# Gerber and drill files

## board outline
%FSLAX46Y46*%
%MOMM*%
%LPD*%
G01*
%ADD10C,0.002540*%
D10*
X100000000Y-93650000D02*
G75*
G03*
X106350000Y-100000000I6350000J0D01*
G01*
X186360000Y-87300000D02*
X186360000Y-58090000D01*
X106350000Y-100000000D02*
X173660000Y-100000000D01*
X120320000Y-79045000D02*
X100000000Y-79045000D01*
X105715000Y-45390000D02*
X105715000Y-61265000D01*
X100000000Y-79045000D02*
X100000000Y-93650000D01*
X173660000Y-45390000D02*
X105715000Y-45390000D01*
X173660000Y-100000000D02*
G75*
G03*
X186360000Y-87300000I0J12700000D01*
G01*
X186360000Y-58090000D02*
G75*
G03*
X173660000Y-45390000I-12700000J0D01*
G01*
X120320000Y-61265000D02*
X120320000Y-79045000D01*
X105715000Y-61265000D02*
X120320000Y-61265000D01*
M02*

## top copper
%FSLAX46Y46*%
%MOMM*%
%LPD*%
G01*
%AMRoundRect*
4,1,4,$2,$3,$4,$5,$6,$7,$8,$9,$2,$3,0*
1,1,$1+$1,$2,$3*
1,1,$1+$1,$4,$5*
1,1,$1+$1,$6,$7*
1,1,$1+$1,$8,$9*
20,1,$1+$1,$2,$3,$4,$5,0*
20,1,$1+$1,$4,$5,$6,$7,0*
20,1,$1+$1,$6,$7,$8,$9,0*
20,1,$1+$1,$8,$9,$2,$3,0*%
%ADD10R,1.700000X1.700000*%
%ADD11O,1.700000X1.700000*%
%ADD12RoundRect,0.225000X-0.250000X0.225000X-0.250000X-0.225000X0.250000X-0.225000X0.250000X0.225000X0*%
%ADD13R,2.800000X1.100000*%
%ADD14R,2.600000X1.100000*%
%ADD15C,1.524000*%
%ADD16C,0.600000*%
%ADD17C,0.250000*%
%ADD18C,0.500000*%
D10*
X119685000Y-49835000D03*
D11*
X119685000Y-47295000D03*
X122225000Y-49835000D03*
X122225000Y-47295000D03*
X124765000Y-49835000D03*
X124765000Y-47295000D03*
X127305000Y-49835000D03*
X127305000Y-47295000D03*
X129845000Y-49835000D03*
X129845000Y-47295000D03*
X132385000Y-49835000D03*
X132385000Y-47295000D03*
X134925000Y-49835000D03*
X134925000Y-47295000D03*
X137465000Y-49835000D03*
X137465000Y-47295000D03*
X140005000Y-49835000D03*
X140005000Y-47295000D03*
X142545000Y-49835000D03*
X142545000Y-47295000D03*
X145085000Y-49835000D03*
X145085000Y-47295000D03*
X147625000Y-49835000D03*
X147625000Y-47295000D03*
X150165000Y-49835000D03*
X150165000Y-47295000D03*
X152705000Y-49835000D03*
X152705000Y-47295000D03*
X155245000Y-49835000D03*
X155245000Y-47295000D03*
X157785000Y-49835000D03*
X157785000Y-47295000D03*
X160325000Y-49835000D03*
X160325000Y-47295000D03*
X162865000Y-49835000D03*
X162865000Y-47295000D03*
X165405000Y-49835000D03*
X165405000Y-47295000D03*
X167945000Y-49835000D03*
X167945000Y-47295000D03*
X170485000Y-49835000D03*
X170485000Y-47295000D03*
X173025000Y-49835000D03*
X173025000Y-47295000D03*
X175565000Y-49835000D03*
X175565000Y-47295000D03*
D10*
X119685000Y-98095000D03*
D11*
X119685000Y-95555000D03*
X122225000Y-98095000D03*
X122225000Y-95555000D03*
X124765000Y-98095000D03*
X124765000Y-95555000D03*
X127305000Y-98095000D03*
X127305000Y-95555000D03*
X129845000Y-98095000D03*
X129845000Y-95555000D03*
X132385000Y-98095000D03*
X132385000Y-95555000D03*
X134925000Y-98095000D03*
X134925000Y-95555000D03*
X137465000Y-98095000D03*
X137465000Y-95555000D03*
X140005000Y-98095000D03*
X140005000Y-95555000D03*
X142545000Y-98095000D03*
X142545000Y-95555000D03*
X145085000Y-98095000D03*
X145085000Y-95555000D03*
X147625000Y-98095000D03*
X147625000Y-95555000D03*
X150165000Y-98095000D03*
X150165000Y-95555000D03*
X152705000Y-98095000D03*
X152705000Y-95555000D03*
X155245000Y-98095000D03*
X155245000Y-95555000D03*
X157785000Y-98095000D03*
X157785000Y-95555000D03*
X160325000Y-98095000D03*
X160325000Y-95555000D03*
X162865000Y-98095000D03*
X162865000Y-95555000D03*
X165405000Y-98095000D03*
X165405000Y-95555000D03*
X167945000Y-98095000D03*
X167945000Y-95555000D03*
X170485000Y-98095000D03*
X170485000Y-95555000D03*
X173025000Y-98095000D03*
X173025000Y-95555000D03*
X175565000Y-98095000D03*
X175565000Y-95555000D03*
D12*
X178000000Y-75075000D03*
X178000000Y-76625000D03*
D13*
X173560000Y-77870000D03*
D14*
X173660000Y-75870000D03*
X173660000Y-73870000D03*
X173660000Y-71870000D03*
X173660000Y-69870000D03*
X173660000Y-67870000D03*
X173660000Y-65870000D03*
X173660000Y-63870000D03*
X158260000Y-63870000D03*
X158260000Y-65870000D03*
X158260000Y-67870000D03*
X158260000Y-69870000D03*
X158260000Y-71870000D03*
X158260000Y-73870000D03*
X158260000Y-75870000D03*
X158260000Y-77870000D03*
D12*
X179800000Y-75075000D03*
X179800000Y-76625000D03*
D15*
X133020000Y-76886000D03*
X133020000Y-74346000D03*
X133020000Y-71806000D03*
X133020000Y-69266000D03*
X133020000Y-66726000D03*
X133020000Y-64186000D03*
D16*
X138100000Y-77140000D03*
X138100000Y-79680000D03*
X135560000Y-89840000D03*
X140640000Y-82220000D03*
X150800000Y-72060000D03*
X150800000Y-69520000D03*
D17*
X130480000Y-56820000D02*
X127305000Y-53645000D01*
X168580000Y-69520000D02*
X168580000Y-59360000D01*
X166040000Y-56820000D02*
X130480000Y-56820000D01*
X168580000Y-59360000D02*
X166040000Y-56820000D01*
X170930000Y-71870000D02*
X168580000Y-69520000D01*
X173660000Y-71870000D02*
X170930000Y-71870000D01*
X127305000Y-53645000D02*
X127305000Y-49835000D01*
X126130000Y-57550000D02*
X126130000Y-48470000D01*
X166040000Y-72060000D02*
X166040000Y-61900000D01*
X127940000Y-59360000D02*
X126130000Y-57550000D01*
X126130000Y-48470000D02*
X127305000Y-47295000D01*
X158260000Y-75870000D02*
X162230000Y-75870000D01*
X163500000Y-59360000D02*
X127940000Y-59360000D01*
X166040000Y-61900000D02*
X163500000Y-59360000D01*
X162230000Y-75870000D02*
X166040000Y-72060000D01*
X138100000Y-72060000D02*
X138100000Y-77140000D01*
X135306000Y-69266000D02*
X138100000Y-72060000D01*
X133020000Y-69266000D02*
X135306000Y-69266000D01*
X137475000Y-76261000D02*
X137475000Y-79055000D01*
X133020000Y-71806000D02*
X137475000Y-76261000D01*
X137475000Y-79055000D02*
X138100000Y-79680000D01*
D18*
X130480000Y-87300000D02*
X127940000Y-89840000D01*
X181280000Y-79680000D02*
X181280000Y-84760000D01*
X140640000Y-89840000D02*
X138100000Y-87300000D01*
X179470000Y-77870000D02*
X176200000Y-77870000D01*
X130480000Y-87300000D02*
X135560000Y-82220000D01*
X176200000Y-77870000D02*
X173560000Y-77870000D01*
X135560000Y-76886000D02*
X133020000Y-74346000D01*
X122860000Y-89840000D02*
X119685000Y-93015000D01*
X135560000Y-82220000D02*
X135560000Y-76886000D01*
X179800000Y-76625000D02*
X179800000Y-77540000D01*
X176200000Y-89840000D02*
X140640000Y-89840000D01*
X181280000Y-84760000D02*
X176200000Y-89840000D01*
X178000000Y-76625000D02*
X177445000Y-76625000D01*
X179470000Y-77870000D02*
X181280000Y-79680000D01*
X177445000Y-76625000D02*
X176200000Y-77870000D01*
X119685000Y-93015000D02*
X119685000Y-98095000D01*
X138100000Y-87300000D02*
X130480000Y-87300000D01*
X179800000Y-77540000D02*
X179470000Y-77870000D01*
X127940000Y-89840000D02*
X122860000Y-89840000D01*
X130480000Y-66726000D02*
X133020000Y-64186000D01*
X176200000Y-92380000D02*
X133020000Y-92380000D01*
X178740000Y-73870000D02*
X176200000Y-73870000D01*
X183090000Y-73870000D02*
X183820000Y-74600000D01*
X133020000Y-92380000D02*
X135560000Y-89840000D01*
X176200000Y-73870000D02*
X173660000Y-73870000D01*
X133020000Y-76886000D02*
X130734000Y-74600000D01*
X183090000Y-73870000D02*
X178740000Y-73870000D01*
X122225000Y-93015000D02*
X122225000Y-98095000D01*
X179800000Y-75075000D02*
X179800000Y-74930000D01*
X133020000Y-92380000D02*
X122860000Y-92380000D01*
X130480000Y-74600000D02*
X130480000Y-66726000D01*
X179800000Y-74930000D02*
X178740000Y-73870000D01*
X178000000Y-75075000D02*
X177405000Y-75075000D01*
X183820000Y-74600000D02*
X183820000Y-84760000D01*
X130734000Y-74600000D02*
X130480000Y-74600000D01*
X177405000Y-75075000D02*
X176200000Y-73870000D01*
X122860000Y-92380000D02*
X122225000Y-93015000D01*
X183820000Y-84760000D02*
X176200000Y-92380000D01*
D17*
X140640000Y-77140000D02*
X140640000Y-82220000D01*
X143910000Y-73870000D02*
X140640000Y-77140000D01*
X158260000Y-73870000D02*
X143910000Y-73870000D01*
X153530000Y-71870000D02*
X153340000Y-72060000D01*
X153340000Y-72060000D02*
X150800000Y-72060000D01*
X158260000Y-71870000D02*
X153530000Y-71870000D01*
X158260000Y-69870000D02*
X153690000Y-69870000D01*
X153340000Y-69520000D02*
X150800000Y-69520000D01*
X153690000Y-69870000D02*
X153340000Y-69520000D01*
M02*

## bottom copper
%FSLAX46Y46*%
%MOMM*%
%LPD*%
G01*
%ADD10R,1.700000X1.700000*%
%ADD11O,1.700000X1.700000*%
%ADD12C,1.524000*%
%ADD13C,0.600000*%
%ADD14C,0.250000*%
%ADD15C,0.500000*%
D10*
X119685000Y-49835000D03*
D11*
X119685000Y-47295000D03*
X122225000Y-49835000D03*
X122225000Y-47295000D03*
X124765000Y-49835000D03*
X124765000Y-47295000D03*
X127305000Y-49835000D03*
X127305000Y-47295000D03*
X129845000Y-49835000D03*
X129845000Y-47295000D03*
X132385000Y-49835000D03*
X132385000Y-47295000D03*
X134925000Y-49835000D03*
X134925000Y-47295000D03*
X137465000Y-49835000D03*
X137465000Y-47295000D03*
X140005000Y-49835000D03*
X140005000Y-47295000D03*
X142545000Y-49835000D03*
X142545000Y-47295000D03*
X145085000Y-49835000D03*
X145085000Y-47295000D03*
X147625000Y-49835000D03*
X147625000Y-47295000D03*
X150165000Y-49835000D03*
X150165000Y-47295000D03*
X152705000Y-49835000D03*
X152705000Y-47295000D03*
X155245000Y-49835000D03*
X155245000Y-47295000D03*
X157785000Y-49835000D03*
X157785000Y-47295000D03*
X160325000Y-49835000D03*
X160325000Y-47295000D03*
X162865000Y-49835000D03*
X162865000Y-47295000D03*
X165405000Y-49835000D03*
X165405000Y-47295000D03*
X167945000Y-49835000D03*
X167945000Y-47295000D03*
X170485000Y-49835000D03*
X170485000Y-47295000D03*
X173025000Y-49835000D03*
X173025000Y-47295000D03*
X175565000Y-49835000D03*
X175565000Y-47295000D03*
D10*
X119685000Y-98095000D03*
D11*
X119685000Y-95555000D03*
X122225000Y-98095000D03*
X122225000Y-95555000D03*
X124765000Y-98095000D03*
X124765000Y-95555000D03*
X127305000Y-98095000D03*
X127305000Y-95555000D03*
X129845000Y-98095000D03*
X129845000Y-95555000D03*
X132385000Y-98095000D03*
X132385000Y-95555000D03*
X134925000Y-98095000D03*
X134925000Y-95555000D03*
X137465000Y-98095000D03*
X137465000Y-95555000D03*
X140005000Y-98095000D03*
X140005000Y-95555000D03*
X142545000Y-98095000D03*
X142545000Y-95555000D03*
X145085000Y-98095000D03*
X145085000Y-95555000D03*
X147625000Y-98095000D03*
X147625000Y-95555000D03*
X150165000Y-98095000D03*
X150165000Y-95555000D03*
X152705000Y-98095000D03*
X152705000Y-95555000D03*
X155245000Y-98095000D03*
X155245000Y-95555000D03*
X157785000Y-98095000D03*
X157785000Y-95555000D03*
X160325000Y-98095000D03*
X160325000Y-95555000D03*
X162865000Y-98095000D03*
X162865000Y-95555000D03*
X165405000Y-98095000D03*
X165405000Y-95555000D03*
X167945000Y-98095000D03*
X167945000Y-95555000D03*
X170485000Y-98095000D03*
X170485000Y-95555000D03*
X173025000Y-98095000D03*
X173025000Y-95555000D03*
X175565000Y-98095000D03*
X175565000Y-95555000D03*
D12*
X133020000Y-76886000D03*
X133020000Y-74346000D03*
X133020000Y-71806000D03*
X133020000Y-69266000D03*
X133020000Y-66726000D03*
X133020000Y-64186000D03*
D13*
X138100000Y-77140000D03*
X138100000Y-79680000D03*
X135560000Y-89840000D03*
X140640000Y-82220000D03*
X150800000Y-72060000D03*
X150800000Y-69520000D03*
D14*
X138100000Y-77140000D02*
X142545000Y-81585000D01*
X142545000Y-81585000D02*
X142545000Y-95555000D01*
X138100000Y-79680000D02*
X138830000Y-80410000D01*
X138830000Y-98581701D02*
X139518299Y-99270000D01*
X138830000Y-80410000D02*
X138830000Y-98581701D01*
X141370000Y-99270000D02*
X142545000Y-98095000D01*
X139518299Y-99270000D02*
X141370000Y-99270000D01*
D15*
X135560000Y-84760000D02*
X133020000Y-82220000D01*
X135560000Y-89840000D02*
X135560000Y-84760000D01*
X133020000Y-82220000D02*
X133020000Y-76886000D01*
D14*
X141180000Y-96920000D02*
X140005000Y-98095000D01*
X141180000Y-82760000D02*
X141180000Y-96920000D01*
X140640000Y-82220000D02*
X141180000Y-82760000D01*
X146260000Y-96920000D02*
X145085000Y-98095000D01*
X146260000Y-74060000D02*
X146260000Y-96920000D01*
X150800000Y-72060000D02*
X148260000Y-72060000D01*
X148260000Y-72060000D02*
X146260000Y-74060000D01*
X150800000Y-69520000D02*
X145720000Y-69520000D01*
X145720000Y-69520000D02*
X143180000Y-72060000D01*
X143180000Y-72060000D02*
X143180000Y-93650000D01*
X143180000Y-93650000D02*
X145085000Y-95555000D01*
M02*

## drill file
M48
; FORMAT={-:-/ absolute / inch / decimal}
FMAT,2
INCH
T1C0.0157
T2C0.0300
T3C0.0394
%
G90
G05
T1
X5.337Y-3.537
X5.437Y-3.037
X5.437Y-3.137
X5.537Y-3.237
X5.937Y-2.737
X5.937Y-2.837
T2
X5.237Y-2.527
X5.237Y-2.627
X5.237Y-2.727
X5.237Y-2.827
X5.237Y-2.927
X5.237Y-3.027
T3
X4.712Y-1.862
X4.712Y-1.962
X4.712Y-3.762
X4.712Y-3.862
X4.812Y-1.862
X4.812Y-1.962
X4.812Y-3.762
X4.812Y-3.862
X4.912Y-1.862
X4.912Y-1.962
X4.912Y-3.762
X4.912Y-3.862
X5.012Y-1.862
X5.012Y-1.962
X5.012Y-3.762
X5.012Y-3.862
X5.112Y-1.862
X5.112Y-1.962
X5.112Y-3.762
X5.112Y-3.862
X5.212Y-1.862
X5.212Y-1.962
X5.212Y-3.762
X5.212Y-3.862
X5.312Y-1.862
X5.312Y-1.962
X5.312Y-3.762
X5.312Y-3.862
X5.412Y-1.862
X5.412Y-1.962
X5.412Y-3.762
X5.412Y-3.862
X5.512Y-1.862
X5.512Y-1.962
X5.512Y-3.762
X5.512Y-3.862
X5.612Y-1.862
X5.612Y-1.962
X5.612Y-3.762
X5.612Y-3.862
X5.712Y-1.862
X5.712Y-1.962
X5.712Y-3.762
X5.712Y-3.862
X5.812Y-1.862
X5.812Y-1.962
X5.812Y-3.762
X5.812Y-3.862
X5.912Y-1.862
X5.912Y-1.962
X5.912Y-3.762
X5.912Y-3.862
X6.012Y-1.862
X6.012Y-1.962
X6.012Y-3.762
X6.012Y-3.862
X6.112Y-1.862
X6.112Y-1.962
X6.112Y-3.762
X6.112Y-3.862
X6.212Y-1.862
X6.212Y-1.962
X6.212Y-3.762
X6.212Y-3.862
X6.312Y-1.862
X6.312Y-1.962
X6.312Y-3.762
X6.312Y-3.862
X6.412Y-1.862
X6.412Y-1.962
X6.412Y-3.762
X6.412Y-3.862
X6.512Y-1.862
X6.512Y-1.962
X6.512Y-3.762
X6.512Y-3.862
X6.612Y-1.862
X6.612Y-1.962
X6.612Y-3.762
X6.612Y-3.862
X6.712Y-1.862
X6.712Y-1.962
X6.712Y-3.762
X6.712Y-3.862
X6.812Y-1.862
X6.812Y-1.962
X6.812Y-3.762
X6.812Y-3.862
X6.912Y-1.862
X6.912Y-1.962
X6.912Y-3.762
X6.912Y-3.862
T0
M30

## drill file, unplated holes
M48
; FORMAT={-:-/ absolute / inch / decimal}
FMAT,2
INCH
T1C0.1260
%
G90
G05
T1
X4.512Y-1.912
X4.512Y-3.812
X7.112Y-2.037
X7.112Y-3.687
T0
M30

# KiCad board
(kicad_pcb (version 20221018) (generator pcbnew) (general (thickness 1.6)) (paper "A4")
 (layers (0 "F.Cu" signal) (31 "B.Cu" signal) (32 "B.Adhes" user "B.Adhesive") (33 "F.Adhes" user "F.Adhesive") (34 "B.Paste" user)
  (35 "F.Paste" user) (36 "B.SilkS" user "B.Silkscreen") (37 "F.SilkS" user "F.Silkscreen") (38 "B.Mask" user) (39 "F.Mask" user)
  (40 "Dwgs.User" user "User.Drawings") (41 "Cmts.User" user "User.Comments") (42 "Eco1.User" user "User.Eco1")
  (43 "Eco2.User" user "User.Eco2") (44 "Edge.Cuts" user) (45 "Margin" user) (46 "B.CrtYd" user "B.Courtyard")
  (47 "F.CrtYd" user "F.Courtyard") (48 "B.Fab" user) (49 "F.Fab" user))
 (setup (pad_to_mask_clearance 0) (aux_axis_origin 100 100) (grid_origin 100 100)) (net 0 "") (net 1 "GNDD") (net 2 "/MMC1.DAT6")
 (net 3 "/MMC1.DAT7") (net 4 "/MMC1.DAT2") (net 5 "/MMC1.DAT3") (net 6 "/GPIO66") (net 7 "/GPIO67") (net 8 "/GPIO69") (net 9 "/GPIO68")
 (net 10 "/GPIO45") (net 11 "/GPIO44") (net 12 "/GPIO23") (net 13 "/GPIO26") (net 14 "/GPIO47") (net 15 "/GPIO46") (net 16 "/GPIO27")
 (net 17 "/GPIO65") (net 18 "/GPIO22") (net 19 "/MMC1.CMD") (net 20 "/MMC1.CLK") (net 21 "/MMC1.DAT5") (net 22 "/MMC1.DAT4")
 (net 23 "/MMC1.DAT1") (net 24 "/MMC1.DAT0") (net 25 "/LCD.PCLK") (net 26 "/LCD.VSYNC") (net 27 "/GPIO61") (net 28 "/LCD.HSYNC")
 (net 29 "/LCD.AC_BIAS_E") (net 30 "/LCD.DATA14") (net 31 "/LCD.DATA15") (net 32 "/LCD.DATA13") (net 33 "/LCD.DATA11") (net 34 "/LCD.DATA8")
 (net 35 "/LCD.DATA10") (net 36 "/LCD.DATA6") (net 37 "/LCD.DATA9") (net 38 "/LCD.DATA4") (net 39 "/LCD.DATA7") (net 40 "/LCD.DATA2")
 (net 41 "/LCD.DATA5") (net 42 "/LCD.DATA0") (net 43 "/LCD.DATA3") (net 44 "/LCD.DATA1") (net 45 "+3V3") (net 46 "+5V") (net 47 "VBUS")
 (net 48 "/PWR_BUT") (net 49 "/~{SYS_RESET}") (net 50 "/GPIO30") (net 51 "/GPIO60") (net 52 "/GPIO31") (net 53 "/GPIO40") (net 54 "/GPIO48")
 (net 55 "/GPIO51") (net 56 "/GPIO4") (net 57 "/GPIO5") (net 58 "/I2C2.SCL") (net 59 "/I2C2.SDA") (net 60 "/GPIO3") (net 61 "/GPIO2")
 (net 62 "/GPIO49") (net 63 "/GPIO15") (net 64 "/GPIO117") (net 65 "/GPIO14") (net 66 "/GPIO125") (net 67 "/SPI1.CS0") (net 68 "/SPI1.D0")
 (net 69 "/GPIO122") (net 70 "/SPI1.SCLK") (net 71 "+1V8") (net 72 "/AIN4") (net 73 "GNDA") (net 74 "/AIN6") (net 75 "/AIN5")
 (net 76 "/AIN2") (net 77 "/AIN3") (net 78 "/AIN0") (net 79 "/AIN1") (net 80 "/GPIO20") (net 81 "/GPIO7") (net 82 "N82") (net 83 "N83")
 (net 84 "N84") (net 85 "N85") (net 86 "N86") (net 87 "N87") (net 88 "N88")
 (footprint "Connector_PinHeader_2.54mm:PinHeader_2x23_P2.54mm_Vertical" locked (layer "F.Cu") (at 119.685 49.835 90)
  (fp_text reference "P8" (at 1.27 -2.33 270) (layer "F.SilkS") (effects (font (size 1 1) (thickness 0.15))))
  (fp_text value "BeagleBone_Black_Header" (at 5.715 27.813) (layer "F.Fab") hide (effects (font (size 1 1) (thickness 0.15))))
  (pad "1" thru_hole rect locked (at 0 0 90) (size 1.7 1.7) (drill 1) (layers "*.Cu" "*.Mask") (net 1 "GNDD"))
  (pad "2" thru_hole oval locked (at 2.54 0 90) (size 1.7 1.7) (drill 1) (layers "*.Cu" "*.Mask") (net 1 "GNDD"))
  (pad "3" thru_hole oval locked (at 0 2.54 90) (size 1.7 1.7) (drill 1) (layers "*.Cu" "*.Mask") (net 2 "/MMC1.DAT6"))
  (pad "4" thru_hole oval locked (at 2.54 2.54 90) (size 1.7 1.7) (drill 1) (layers "*.Cu" "*.Mask") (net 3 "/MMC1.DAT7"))
  (pad "5" thru_hole oval locked (at 0 5.08 90) (size 1.7 1.7) (drill 1) (layers "*.Cu" "*.Mask") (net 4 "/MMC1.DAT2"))
  (pad "6" thru_hole oval locked (at 2.54 5.08 90) (size 1.7 1.7) (drill 1) (layers "*.Cu" "*.Mask") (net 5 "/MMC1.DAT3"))
  (pad "7" thru_hole oval locked (at 0 7.62 90) (size 1.7 1.7) (drill 1) (layers "*.Cu" "*.Mask") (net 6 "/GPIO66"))
  (pad "8" thru_hole oval locked (at 2.54 7.62 90) (size 1.7 1.7) (drill 1) (layers "*.Cu" "*.Mask") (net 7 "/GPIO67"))
  (pad "9" thru_hole oval locked (at 0 10.16 90) (size 1.7 1.7) (drill 1) (layers "*.Cu" "*.Mask") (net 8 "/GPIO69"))
  (pad "10" thru_hole oval locked (at 2.54 10.16 90) (size 1.7 1.7) (drill 1) (layers "*.Cu" "*.Mask") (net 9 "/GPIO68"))
  (pad "11" thru_hole oval locked (at 0 12.7 90) (size 1.7 1.7) (drill 1) (layers "*.Cu" "*.Mask") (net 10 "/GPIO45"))
  (pad "12" thru_hole oval locked (at 2.54 12.7 90) (size 1.7 1.7) (drill 1) (layers "*.Cu" "*.Mask") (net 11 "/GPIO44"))
  (pad "13" thru_hole oval locked (at 0 15.24 90) (size 1.7 1.7) (drill 1) (layers "*.Cu" "*.Mask") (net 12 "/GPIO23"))
  (pad "14" thru_hole oval locked (at 2.54 15.24 90) (size 1.7 1.7) (drill 1) (layers "*.Cu" "*.Mask") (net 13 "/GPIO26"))
  (pad "15" thru_hole oval locked (at 0 17.78 90) (size 1.7 1.7) (drill 1) (layers "*.Cu" "*.Mask") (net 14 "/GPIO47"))
  (pad "16" thru_hole oval locked (at 2.54 17.78 90) (size 1.7 1.7) (drill 1) (layers "*.Cu" "*.Mask") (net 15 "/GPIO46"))
  (pad "17" thru_hole oval locked (at 0 20.32 90) (size 1.7 1.7) (drill 1) (layers "*.Cu" "*.Mask") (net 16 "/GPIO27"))
  (pad "18" thru_hole oval locked (at 2.54 20.32 90) (size 1.7 1.7) (drill 1) (layers "*.Cu" "*.Mask") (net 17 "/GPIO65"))
  (pad "19" thru_hole oval locked (at 0 22.86 90) (size 1.7 1.7) (drill 1) (layers "*.Cu" "*.Mask") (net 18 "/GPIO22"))
  (pad "20" thru_hole oval locked (at 2.54 22.86 90) (size 1.7 1.7) (drill 1) (layers "*.Cu" "*.Mask") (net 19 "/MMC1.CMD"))
  (pad "21" thru_hole oval locked (at 0 25.4 90) (size 1.7 1.7) (drill 1) (layers "*.Cu" "*.Mask") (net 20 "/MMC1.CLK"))
  (pad "22" thru_hole oval locked (at 2.54 25.4 90) (size 1.7 1.7) (drill 1) (layers "*.Cu" "*.Mask") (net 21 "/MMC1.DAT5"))
  (pad "23" thru_hole oval locked (at 0 27.94 90) (size 1.7 1.7) (drill 1) (layers "*.Cu" "*.Mask") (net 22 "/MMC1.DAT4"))
  (pad "24" thru_hole oval locked (at 2.54 27.94 90) (size 1.7 1.7) (drill 1) (layers "*.Cu" "*.Mask") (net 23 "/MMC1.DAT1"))
  (pad "25" thru_hole oval locked (at 0 30.48 90) (size 1.7 1.7) (drill 1) (layers "*.Cu" "*.Mask") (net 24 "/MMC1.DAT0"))
  (pad "26" thru_hole oval locked (at 2.54 30.48 90) (size 1.7 1.7) (drill 1) (layers "*.Cu" "*.Mask") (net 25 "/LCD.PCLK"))
  (pad "27" thru_hole oval locked (at 0 33.02 90) (size 1.7 1.7) (drill 1) (layers "*.Cu" "*.Mask") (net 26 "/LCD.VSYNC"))
  (pad "28" thru_hole oval locked (at 2.54 33.02 90) (size 1.7 1.7) (drill 1) (layers "*.Cu" "*.Mask") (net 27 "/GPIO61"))
  (pad "29" thru_hole oval locked (at 0 35.56 90) (size 1.7 1.7) (drill 1) (layers "*.Cu" "*.Mask") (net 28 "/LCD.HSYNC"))
  (pad "30" thru_hole oval locked (at 2.54 35.56 90) (size 1.7 1.7) (drill 1) (layers "*.Cu" "*.Mask") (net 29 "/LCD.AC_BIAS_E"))
  (pad "31" thru_hole oval locked (at 0 38.1 90) (size 1.7 1.7) (drill 1) (layers "*.Cu" "*.Mask") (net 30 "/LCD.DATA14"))
  (pad "32" thru_hole oval locked (at 2.54 38.1 90) (size 1.7 1.7) (drill 1) (layers "*.Cu" "*.Mask") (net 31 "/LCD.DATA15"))
  (pad "33" thru_hole oval locked (at 0 40.64 90) (size 1.7 1.7) (drill 1) (layers "*.Cu" "*.Mask") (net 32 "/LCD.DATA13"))
  (pad "34" thru_hole oval locked (at 2.54 40.64 90) (size 1.7 1.7) (drill 1) (layers "*.Cu" "*.Mask") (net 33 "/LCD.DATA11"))
  (pad "35" thru_hole oval locked (at 0 43.18 90) (size 1.7 1.7) (drill 1) (layers "*.Cu" "*.Mask") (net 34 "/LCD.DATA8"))
  (pad "36" thru_hole oval locked (at 2.54 43.18 90) (size 1.7 1.7) (drill 1) (layers "*.Cu" "*.Mask") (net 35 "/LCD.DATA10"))
  (pad "37" thru_hole oval locked (at 0 45.72 90) (size 1.7 1.7) (drill 1) (layers "*.Cu" "*.Mask") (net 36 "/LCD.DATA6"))
  (pad "38" thru_hole oval locked (at 2.54 45.72 90) (size 1.7 1.7) (drill 1) (layers "*.Cu" "*.Mask") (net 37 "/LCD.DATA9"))
  (pad "39" thru_hole oval locked (at 0 48.26 90) (size 1.7 1.7) (drill 1) (layers "*.Cu" "*.Mask") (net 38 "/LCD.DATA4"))
  (pad "40" thru_hole oval locked (at 2.54 48.26 90) (size 1.7 1.7) (drill 1) (layers "*.Cu" "*.Mask") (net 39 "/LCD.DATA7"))
  (pad "41" thru_hole oval locked (at 0 50.8 90) (size 1.7 1.7) (drill 1) (layers "*.Cu" "*.Mask") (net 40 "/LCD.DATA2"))
  (pad "42" thru_hole oval locked (at 2.54 50.8 90) (size 1.7 1.7) (drill 1) (layers "*.Cu" "*.Mask") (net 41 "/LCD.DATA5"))
  (pad "43" thru_hole oval locked (at 0 53.34 90) (size 1.7 1.7) (drill 1) (layers "*.Cu" "*.Mask") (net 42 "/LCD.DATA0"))
  (pad "44" thru_hole oval locked (at 2.54 53.34 90) (size 1.7 1.7) (drill 1) (layers "*.Cu" "*.Mask") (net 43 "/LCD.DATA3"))
  (pad "45" thru_hole oval locked (at 0 55.88 90) (size 1.7 1.7) (drill 1) (layers "*.Cu" "*.Mask") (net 1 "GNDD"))
  (pad "46" thru_hole oval locked (at 2.54 55.88 90) (size 1.7 1.7) (drill 1) (layers "*.Cu" "*.Mask") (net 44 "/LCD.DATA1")))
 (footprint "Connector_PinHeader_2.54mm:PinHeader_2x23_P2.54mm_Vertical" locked (layer "F.Cu") (at 119.685 98.095 90)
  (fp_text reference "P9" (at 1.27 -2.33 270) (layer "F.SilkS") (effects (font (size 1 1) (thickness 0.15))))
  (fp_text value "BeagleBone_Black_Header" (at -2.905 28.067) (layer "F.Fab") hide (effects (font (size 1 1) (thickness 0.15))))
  (pad "1" thru_hole rect locked (at 0 0 90) (size 1.7 1.7) (drill 1) (layers "*.Cu" "*.Mask") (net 1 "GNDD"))
  (pad "2" thru_hole oval locked (at 2.54 0 90) (size 1.7 1.7) (drill 1) (layers "*.Cu" "*.Mask") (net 1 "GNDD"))
  (pad "3" thru_hole oval locked (at 0 2.54 90) (size 1.7 1.7) (drill 1) (layers "*.Cu" "*.Mask") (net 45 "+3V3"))
  (pad "4" thru_hole oval locked (at 2.54 2.54 90) (size 1.7 1.7) (drill 1) (layers "*.Cu" "*.Mask") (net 45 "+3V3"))
  (pad "5" thru_hole oval locked (at 0 5.08 90) (size 1.7 1.7) (drill 1) (layers "*.Cu" "*.Mask") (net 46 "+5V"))
  (pad "6" thru_hole oval locked (at 2.54 5.08 90) (size 1.7 1.7) (drill 1) (layers "*.Cu" "*.Mask") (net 46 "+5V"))
  (pad "7" thru_hole oval locked (at 0 7.62 90) (size 1.7 1.7) (drill 1) (layers "*.Cu" "*.Mask") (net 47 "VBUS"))
  (pad "8" thru_hole oval locked (at 2.54 7.62 90) (size 1.7 1.7) (drill 1) (layers "*.Cu" "*.Mask") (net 47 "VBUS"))
  (pad "9" thru_hole oval locked (at 0 10.16 90) (size 1.7 1.7) (drill 1) (layers "*.Cu" "*.Mask") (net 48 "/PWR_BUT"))
  (pad "10" thru_hole oval locked (at 2.54 10.16 90) (size 1.7 1.7) (drill 1) (layers "*.Cu" "*.Mask") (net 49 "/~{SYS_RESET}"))
  (pad "11" thru_hole oval locked (at 0 12.7 90) (size 1.7 1.7) (drill 1) (layers "*.Cu" "*.Mask") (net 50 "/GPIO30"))
  (pad "12" thru_hole oval locked (at 2.54 12.7 90) (size 1.7 1.7) (drill 1) (layers "*.Cu" "*.Mask") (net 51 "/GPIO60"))
  (pad "13" thru_hole oval locked (at 0 15.24 90) (size 1.7 1.7) (drill 1) (layers "*.Cu" "*.Mask") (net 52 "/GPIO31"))
  (pad "14" thru_hole oval locked (at 2.54 15.24 90) (size 1.7 1.7) (drill 1) (layers "*.Cu" "*.Mask") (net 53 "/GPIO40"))
  (pad "15" thru_hole oval locked (at 0 17.78 90) (size 1.7 1.7) (drill 1) (layers "*.Cu" "*.Mask") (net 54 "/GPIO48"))
  (pad "16" thru_hole oval locked (at 2.54 17.78 90) (size 1.7 1.7) (drill 1) (layers "*.Cu" "*.Mask") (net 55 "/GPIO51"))
  (pad "17" thru_hole oval locked (at 0 20.32 90) (size 1.7 1.7) (drill 1) (layers "*.Cu" "*.Mask") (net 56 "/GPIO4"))
  (pad "18" thru_hole oval locked (at 2.54 20.32 90) (size 1.7 1.7) (drill 1) (layers "*.Cu" "*.Mask") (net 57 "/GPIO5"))
  (pad "19" thru_hole oval locked (at 0 22.86 90) (size 1.7 1.7) (drill 1) (layers "*.Cu" "*.Mask") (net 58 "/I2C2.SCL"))
  (pad "20" thru_hole oval locked (at 2.54 22.86 90) (size 1.7 1.7) (drill 1) (layers "*.Cu" "*.Mask") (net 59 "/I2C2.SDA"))
  (pad "21" thru_hole oval locked (at 0 25.4 90) (size 1.7 1.7) (drill 1) (layers "*.Cu" "*.Mask") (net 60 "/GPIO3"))
  (pad "22" thru_hole oval locked (at 2.54 25.4 90) (size 1.7 1.7) (drill 1) (layers "*.Cu" "*.Mask") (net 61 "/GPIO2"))
  (pad "23" thru_hole oval locked (at 0 27.94 90) (size 1.7 1.7) (drill 1) (layers "*.Cu" "*.Mask") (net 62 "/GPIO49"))
  (pad "24" thru_hole oval locked (at 2.54 27.94 90) (size 1.7 1.7) (drill 1) (layers "*.Cu" "*.Mask") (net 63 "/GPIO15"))
  (pad "25" thru_hole oval locked (at 0 30.48 90) (size 1.7 1.7) (drill 1) (layers "*.Cu" "*.Mask") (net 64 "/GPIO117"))
  (pad "26" thru_hole oval locked (at 2.54 30.48 90) (size 1.7 1.7) (drill 1) (layers "*.Cu" "*.Mask") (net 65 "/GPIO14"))
  (pad "27" thru_hole oval locked (at 0 33.02 90) (size 1.7 1.7) (drill 1) (layers "*.Cu" "*.Mask") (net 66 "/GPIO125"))
  (pad "28" thru_hole oval locked (at 2.54 33.02 90) (size 1.7 1.7) (drill 1) (layers "*.Cu" "*.Mask") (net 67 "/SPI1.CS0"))
  (pad "29" thru_hole oval locked (at 0 35.56 90) (size 1.7 1.7) (drill 1) (layers "*.Cu" "*.Mask") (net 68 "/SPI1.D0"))
  (pad "30" thru_hole oval locked (at 2.54 35.56 90) (size 1.7 1.7) (drill 1) (layers "*.Cu" "*.Mask") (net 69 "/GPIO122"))
  (pad "31" thru_hole oval locked (at 0 38.1 90) (size 1.7 1.7) (drill 1) (layers "*.Cu" "*.Mask") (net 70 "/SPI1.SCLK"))
  (pad "32" thru_hole oval locked (at 2.54 38.1 90) (size 1.7 1.7) (drill 1) (layers "*.Cu" "*.Mask") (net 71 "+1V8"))
  (pad "33" thru_hole oval locked (at 0 40.64 90) (size 1.7 1.7) (drill 1) (layers "*.Cu" "*.Mask") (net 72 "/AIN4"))
  (pad "34" thru_hole oval locked (at 2.54 40.64 90) (size 1.7 1.7) (drill 1) (layers "*.Cu" "*.Mask") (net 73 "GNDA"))
  (pad "35" thru_hole oval locked (at 0 43.18 90) (size 1.7 1.7) (drill 1) (layers "*.Cu" "*.Mask") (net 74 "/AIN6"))
  (pad "36" thru_hole oval locked (at 2.54 43.18 90) (size 1.7 1.7) (drill 1) (layers "*.Cu" "*.Mask") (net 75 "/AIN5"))
  (pad "37" thru_hole oval locked (at 0 45.72 90) (size 1.7 1.7) (drill 1) (layers "*.Cu" "*.Mask") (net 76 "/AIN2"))
  (pad "38" thru_hole oval locked (at 2.54 45.72 90) (size 1.7 1.7) (drill 1) (layers "*.Cu" "*.Mask") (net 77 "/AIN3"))
  (pad "39" thru_hole oval locked (at 0 48.26 90) (size 1.7 1.7) (drill 1) (layers "*.Cu" "*.Mask") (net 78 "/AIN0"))
  (pad "40" thru_hole oval locked (at 2.54 48.26 90) (size 1.7 1.7) (drill 1) (layers "*.Cu" "*.Mask") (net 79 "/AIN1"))
  (pad "41" thru_hole oval locked (at 0 50.8 90) (size 1.7 1.7) (drill 1) (layers "*.Cu" "*.Mask") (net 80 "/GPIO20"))
  (pad "42" thru_hole oval locked (at 2.54 50.8 90) (size 1.7 1.7) (drill 1) (layers "*.Cu" "*.Mask") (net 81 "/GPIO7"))
  (pad "43" thru_hole oval locked (at 0 53.34 90) (size 1.7 1.7) (drill 1) (layers "*.Cu" "*.Mask") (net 1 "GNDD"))
  (pad "44" thru_hole oval locked (at 2.54 53.34 90) (size 1.7 1.7) (drill 1) (layers "*.Cu" "*.Mask") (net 1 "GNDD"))
  (pad "45" thru_hole oval locked (at 0 55.88 90) (size 1.7 1.7) (drill 1) (layers "*.Cu" "*.Mask") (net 1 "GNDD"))
  (pad "46" thru_hole oval locked (at 2.54 55.88 90) (size 1.7 1.7) (drill 1) (layers "*.Cu" "*.Mask") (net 1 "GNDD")))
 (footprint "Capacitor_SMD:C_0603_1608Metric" (layer "F.Cu") (at 178 75.85 -90)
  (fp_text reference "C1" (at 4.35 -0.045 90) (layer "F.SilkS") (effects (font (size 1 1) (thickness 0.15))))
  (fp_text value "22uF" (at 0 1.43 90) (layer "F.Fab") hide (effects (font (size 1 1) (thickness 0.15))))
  (pad "1" smd roundrect (at -0.775 0 270) (size 0.9 0.95) (layers "F.Cu" "F.Paste" "F.Mask") (roundrect_rratio 0.25) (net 45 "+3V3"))
  (pad "2" smd roundrect (at 0.775 0 270) (size 0.9 0.95) (layers "F.Cu" "F.Paste" "F.Mask") (roundrect_rratio 0.25) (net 1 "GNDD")))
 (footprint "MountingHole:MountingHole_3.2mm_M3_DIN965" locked (layer "F.Cu") (at 180.645 51.74)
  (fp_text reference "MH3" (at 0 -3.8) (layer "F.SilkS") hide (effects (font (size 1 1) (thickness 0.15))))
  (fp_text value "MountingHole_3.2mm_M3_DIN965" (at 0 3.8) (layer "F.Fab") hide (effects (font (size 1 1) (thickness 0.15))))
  (pad "" np_thru_hole circle locked (at 0 0) (size 3.2 3.2) (drill 3.2) (layers "*.Cu" "*.Mask")))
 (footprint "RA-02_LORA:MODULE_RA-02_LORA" (layer "F.Cu") (at 165.96 70.87 180)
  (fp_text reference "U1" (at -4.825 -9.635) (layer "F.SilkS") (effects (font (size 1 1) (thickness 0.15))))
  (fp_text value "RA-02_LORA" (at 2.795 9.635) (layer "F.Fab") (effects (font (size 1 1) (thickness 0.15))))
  (pad "1" smd rect (at -7.6 -7 180) (size 2.8 1.1) (layers "F.Cu" "F.Paste" "F.Mask") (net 1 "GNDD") (solder_mask_margin 0.102))
  (pad "2" smd rect (at -7.7 -5 180) (size 2.6 1.1) (layers "F.Cu" "F.Paste" "F.Mask") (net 1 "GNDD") (solder_mask_margin 0.102))
  (pad "3" smd rect (at -7.7 -3 180) (size 2.6 1.1) (layers "F.Cu" "F.Paste" "F.Mask") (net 45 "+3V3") (solder_mask_margin 0.102))
  (pad "4" smd rect (at -7.7 -1 180) (size 2.6 1.1) (layers "F.Cu" "F.Paste" "F.Mask") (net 6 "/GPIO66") (solder_mask_margin 0.102))
  (pad "5" smd rect (at -7.7 1 180) (size 2.6 1.1) (layers "F.Cu" "F.Paste" "F.Mask") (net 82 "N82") (solder_mask_margin 0.102))
  (pad "6" smd rect (at -7.7 3 180) (size 2.6 1.1) (layers "F.Cu" "F.Paste" "F.Mask") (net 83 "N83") (solder_mask_margin 0.102))
  (pad "7" smd rect (at -7.7 5 180) (size 2.6 1.1) (layers "F.Cu" "F.Paste" "F.Mask") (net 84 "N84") (solder_mask_margin 0.102))
  (pad "8" smd rect (at -7.7 7 180) (size 2.6 1.1) (layers "F.Cu" "F.Paste" "F.Mask") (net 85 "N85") (solder_mask_margin 0.102))
  (pad "9" smd rect (at 7.7 7) (size 2.6 1.1) (layers "F.Cu" "F.Paste" "F.Mask") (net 1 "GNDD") (solder_mask_margin 0.102))
  (pad "10" smd rect (at 7.7 5) (size 2.6 1.1) (layers "F.Cu" "F.Paste" "F.Mask") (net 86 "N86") (solder_mask_margin 0.102))
  (pad "11" smd rect (at 7.7 3) (size 2.6 1.1) (layers "F.Cu" "F.Paste" "F.Mask") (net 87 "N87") (solder_mask_margin 0.102))
  (pad "12" smd rect (at 7.7 1) (size 2.6 1.1) (layers "F.Cu" "F.Paste" "F.Mask") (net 61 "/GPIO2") (solder_mask_margin 0.102))
  (pad "13" smd rect (at 7.7 -1) (size 2.6 1.1) (layers "F.Cu" "F.Paste" "F.Mask") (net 60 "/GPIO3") (solder_mask_margin 0.102))
  (pad "14" smd rect (at 7.7 -3) (size 2.6 1.1) (layers "F.Cu" "F.Paste" "F.Mask") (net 56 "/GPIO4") (solder_mask_margin 0.102))
  (pad "15" smd rect (at 7.7 -5) (size 2.6 1.1) (layers "F.Cu" "F.Paste" "F.Mask") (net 7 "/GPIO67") (solder_mask_margin 0.102))
  (pad "16" smd rect (at 7.7 -7) (size 2.6 1.1) (layers "F.Cu" "F.Paste" "F.Mask") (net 1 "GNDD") (solder_mask_margin 0.102)))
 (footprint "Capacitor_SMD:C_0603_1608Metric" (layer "F.Cu") (at 179.8 75.85 -90)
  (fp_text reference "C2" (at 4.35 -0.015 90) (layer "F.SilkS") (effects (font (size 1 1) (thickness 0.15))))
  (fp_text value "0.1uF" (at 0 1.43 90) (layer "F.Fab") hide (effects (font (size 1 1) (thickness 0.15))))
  (pad "1" smd roundrect (at -0.775 0 270) (size 0.9 0.95) (layers "F.Cu" "F.Paste" "F.Mask") (roundrect_rratio 0.25) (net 45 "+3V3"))
  (pad "2" smd roundrect (at 0.775 0 270) (size 0.9 0.95) (layers "F.Cu" "F.Paste" "F.Mask") (roundrect_rratio 0.25) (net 1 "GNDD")))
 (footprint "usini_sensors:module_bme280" (layer "F.Cu") (at 127.94 64.44 180)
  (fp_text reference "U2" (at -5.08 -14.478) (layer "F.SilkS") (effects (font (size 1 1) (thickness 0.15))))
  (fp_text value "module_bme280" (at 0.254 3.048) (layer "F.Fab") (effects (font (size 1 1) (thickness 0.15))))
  (pad "1" thru_hole circle (at -5.08 -12.446 180) (size 1.524 1.524) (drill 0.762) (layers "*.Cu" "*.Mask") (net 45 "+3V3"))
  (pad "2" thru_hole circle (at -5.08 -9.906 180) (size 1.524 1.524) (drill 0.762) (layers "*.Cu" "*.Mask") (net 1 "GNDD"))
  (pad "3" thru_hole circle (at -5.08 -7.366 180) (size 1.524 1.524) (drill 0.762) (layers "*.Cu" "*.Mask") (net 58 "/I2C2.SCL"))
  (pad "4" thru_hole circle (at -5.08 -4.826 180) (size 1.524 1.524) (drill 0.762) (layers "*.Cu" "*.Mask") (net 59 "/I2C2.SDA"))
  (pad "5" thru_hole circle (at -5.08 -2.286 180) (size 1.524 1.524) (drill 0.762) (layers "*.Cu" "*.Mask") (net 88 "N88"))
  (pad "6" thru_hole circle (at -5.08 0.254 180) (size 1.524 1.524) (drill 0.762) (layers "*.Cu" "*.Mask") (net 45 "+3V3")))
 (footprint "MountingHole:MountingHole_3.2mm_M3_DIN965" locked (layer "F.Cu") (at 180.645 93.65)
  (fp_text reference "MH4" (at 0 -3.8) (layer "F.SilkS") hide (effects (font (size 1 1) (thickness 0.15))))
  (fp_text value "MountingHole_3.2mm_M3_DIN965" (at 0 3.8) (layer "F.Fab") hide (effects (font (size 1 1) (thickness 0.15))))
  (pad "" np_thru_hole circle locked (at 0 0) (size 3.2 3.2) (drill 3.2) (layers "*.Cu" "*.Mask")))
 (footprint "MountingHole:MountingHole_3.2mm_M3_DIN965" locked (layer "F.Cu") (at 114.605 48.565)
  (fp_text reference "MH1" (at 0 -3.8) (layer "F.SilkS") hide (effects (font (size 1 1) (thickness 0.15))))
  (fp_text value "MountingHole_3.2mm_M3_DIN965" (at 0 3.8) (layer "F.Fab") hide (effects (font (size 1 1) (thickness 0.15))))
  (pad "" np_thru_hole circle locked (at 0 0) (size 3.2 3.2) (drill 3.2) (layers "*.Cu" "*.Mask")))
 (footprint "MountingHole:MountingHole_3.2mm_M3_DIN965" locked (layer "F.Cu") (at 114.605 96.825)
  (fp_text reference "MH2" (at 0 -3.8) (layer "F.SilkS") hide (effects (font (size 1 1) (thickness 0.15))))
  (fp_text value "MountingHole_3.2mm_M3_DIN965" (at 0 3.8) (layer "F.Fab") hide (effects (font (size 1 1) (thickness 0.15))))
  (pad "" np_thru_hole circle locked (at 0 0) (size 3.2 3.2) (drill 3.2) (layers "*.Cu" "*.Mask")))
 (gr_arc locked (start 106.35 100) (mid 101.859872 98.140128) (end 100 93.65) (stroke (width 0.00254) (type solid)) (layer "Edge.Cuts"))
 (gr_line locked (start 186.36 87.3) (end 186.36 58.09) (stroke (width 0.00254) (type solid)) (layer "Edge.Cuts"))
 (gr_line locked (start 106.35 100) (end 173.66 100) (stroke (width 0.00254) (type solid)) (layer "Edge.Cuts"))
 (gr_line locked (start 120.32 79.045) (end 100 79.045) (stroke (width 0.00254) (type solid)) (layer "Edge.Cuts"))
 (gr_line locked (start 105.715 45.39) (end 105.715 61.265) (stroke (width 0.00254) (type solid)) (layer "Edge.Cuts"))
 (gr_line locked (start 100 79.045) (end 100 93.65) (stroke (width 0.00254) (type solid)) (layer "Edge.Cuts"))
 (gr_line locked (start 173.66 45.39) (end 105.715 45.39) (stroke (width 0.00254) (type solid)) (layer "Edge.Cuts"))
 (gr_arc locked (start 186.36 87.3) (mid 182.640256 96.280256) (end 173.66 100) (stroke (width 0.00254) (type solid)) (layer "Edge.Cuts"))
 (gr_arc locked (start 173.66 45.39) (mid 182.640256 49.109744) (end 186.36 58.09) (stroke (width 0.00254) (type solid)) (layer "Edge.Cuts"))
 (gr_line locked (start 120.32 61.265) (end 120.32 79.045) (stroke (width 0.00254) (type solid)) (layer "Edge.Cuts"))
 (gr_line locked (start 105.715 61.265) (end 120.32 61.265) (stroke (width 0.00254) (type solid)) (layer "Edge.Cuts"))
 (segment (start 130.48 56.82) (end 127.305 53.645) (width 0.25) (layer "F.Cu") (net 6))
 (segment (start 168.58 69.52) (end 168.58 59.36) (width 0.25) (layer "F.Cu") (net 6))
 (segment (start 166.04 56.82) (end 130.48 56.82) (width 0.25) (layer "F.Cu") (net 6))
 (segment (start 168.58 59.36) (end 166.04 56.82) (width 0.25) (layer "F.Cu") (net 6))
 (segment (start 170.93 71.87) (end 168.58 69.52) (width 0.25) (layer "F.Cu") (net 6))
 (segment (start 173.66 71.87) (end 170.93 71.87) (width 0.25) (layer "F.Cu") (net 6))
 (segment (start 127.305 53.645) (end 127.305 49.835) (width 0.25) (layer "F.Cu") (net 6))
 (segment (start 126.13 57.55) (end 126.13 48.47) (width 0.25) (layer "F.Cu") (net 7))
 (segment (start 166.04 72.06) (end 166.04 61.9) (width 0.25) (layer "F.Cu") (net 7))
 (segment (start 127.94 59.36) (end 126.13 57.55) (width 0.25) (layer "F.Cu") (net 7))
 (segment (start 126.13 48.47) (end 127.305 47.295) (width 0.25) (layer "F.Cu") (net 7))
 (segment (start 158.26 75.87) (end 162.23 75.87) (width 0.25) (layer "F.Cu") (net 7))
 (segment (start 163.5 59.36) (end 127.94 59.36) (width 0.25) (layer "F.Cu") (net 7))
 (segment (start 166.04 61.9) (end 163.5 59.36) (width 0.25) (layer "F.Cu") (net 7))
 (segment (start 162.23 75.87) (end 166.04 72.06) (width 0.25) (layer "F.Cu") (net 7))
 (segment (start 138.1 72.06) (end 138.1 77.14) (width 0.25) (layer "F.Cu") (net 59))
 (segment (start 135.306 69.266) (end 138.1 72.06) (width 0.25) (layer "F.Cu") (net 59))
 (segment (start 133.02 69.266) (end 135.306 69.266) (width 0.25) (layer "F.Cu") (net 59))
 (via (at 138.1 77.14) (size 0.6) (drill 0.4) (layers "F.Cu" "B.Cu") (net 59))
 (segment (start 138.1 77.14) (end 142.545 81.585) (width 0.25) (layer "B.Cu") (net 59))
 (segment (start 142.545 81.585) (end 142.545 95.555) (width 0.25) (layer "B.Cu") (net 59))
 (segment (start 137.475 76.261) (end 137.475 79.055) (width 0.25) (layer "F.Cu") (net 58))
 (segment (start 133.02 71.806) (end 137.475 76.261) (width 0.25) (layer "F.Cu") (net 58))
 (segment (start 137.475 79.055) (end 138.1 79.68) (width 0.25) (layer "F.Cu") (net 58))
 (via (at 138.1 79.68) (size 0.6) (drill 0.4) (layers "F.Cu" "B.Cu") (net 58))
 (segment (start 138.1 79.68) (end 138.83 80.41) (width 0.25) (layer "B.Cu") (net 58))
 (segment (start 138.83 98.581701) (end 139.518299 99.27) (width 0.25) (layer "B.Cu") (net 58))
 (segment (start 138.83 80.41) (end 138.83 98.581701) (width 0.25) (layer "B.Cu") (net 58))
 (segment (start 141.37 99.27) (end 142.545 98.095) (width 0.25) (layer "B.Cu") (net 58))
 (segment (start 139.518299 99.27) (end 141.37 99.27) (width 0.25) (layer "B.Cu") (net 58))
 (segment (start 130.48 87.3) (end 127.94 89.84) (width 0.5) (layer "F.Cu") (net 1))
 (segment (start 181.28 79.68) (end 181.28 84.76) (width 0.5) (layer "F.Cu") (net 1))
 (segment (start 140.64 89.84) (end 138.1 87.3) (width 0.5) (layer "F.Cu") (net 1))
 (segment (start 179.47 77.87) (end 176.2 77.87) (width 0.5) (layer "F.Cu") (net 1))
 (segment (start 130.48 87.3) (end 135.56 82.22) (width 0.5) (layer "F.Cu") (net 1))
 (segment (start 176.2 77.87) (end 173.56 77.87) (width 0.5) (layer "F.Cu") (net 1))
 (segment (start 135.56 76.886) (end 133.02 74.346) (width 0.5) (layer "F.Cu") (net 1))
 (segment (start 122.86 89.84) (end 119.685 93.015) (width 0.5) (layer "F.Cu") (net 1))
 (segment (start 135.56 82.22) (end 135.56 76.886) (width 0.5) (layer "F.Cu") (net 1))
 (segment (start 179.8 76.625) (end 179.8 77.54) (width 0.5) (layer "F.Cu") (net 1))
 (segment (start 176.2 89.84) (end 140.64 89.84) (width 0.5) (layer "F.Cu") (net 1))
 (segment (start 181.28 84.76) (end 176.2 89.84) (width 0.5) (layer "F.Cu") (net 1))
 (segment (start 178 76.625) (end 177.445 76.625) (width 0.5) (layer "F.Cu") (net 1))
 (segment (start 179.47 77.87) (end 181.28 79.68) (width 0.5) (layer "F.Cu") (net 1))
 (segment (start 177.445 76.625) (end 176.2 77.87) (width 0.5) (layer "F.Cu") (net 1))
 (segment (start 119.685 93.015) (end 119.685 98.095) (width 0.5) (layer "F.Cu") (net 1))
 (segment (start 138.1 87.3) (end 130.48 87.3) (width 0.5) (layer "F.Cu") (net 1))
 (segment (start 179.8 77.54) (end 179.47 77.87) (width 0.5) (layer "F.Cu") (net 1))
 (segment (start 127.94 89.84) (end 122.86 89.84) (width 0.5) (layer "F.Cu") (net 1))
 (segment (start 130.48 66.726) (end 133.02 64.186) (width 0.5) (layer "F.Cu") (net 45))
 (segment (start 176.2 92.38) (end 133.02 92.38) (width 0.5) (layer "F.Cu") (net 45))
 (segment (start 178.74 73.87) (end 176.2 73.87) (width 0.5) (layer "F.Cu") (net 45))
 (segment (start 183.09 73.87) (end 183.82 74.6) (width 0.5) (layer "F.Cu") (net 45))
 (segment (start 133.02 92.38) (end 135.56 89.84) (width 0.5) (layer "F.Cu") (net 45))
 (segment (start 176.2 73.87) (end 173.66 73.87) (width 0.5) (layer "F.Cu") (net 45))
 (segment (start 133.02 76.886) (end 130.734 74.6) (width 0.5) (layer "F.Cu") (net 45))
 (segment (start 183.09 73.87) (end 178.74 73.87) (width 0.5) (layer "F.Cu") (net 45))
 (segment (start 122.225 93.015) (end 122.225 98.095) (width 0.5) (layer "F.Cu") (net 45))
 (segment (start 179.8 75.075) (end 179.8 74.93) (width 0.5) (layer "F.Cu") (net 45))
 (segment (start 133.02 92.38) (end 122.86 92.38) (width 0.5) (layer "F.Cu") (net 45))
 (segment (start 130.48 74.6) (end 130.48 66.726) (width 0.5) (layer "F.Cu") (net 45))
 (segment (start 179.8 74.93) (end 178.74 73.87) (width 0.5) (layer "F.Cu") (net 45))
 (segment (start 178 75.075) (end 177.405 75.075) (width 0.5) (layer "F.Cu") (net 45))
 (segment (start 183.82 74.6) (end 183.82 84.76) (width 0.5) (layer "F.Cu") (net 45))
 (segment (start 130.734 74.6) (end 130.48 74.6) (width 0.5) (layer "F.Cu") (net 45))
 (segment (start 177.405 75.075) (end 176.2 73.87) (width 0.5) (layer "F.Cu") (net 45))
 (segment (start 122.86 92.38) (end 122.225 93.015) (width 0.5) (layer "F.Cu") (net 45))
 (segment (start 183.82 84.76) (end 176.2 92.38) (width 0.5) (layer "F.Cu") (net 45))
 (via (at 135.56 89.84) (size 0.6) (drill 0.4) (layers "F.Cu" "B.Cu") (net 45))
 (segment (start 135.56 84.76) (end 133.02 82.22) (width 0.5) (layer "B.Cu") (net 45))
 (segment (start 135.56 89.84) (end 135.56 84.76) (width 0.5) (layer "B.Cu") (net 45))
 (segment (start 133.02 82.22) (end 133.02 76.886) (width 0.5) (layer "B.Cu") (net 45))
 (segment (start 140.64 77.14) (end 140.64 82.22) (width 0.25) (layer "F.Cu") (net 56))
 (segment (start 143.91 73.87) (end 140.64 77.14) (width 0.25) (layer "F.Cu") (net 56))
 (segment (start 158.26 73.87) (end 143.91 73.87) (width 0.25) (layer "F.Cu") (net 56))
 (via (at 140.64 82.22) (size 0.6) (drill 0.4) (layers "F.Cu" "B.Cu") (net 56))
 (segment (start 141.18 96.92) (end 140.005 98.095) (width 0.25) (layer "B.Cu") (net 56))
 (segment (start 141.18 82.76) (end 141.18 96.92) (width 0.25) (layer "B.Cu") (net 56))
 (segment (start 140.64 82.22) (end 141.18 82.76) (width 0.25) (layer "B.Cu") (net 56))
 (segment (start 153.53 71.87) (end 153.34 72.06) (width 0.25) (layer "F.Cu") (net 60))
 (segment (start 153.34 72.06) (end 150.8 72.06) (width 0.25) (layer "F.Cu") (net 60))
 (segment (start 158.26 71.87) (end 153.53 71.87) (width 0.25) (layer "F.Cu") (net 60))
 (via (at 150.8 72.06) (size 0.6) (drill 0.4) (layers "F.Cu" "B.Cu") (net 60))
 (segment (start 146.26 96.92) (end 145.085 98.095) (width 0.25) (layer "B.Cu") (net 60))
 (segment (start 146.26 74.06) (end 146.26 96.92) (width 0.25) (layer "B.Cu") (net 60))
 (segment (start 150.8 72.06) (end 148.26 72.06) (width 0.25) (layer "B.Cu") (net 60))
 (segment (start 148.26 72.06) (end 146.26 74.06) (width 0.25) (layer "B.Cu") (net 60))
 (segment (start 158.26 69.87) (end 153.69 69.87) (width 0.25) (layer "F.Cu") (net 61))
 (segment (start 153.34 69.52) (end 150.8 69.52) (width 0.25) (layer "F.Cu") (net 61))
 (segment (start 153.69 69.87) (end 153.34 69.52) (width 0.25) (layer "F.Cu") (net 61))
 (via (at 150.8 69.52) (size 0.6) (drill 0.4) (layers "F.Cu" "B.Cu") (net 61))
 (segment (start 150.8 69.52) (end 145.72 69.52) (width 0.25) (layer "B.Cu") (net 61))
 (segment (start 145.72 69.52) (end 143.18 72.06) (width 0.25) (layer "B.Cu") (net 61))
 (segment (start 143.18 72.06) (end 143.18 93.65) (width 0.25) (layer "B.Cu") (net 61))
 (segment (start 143.18 93.65) (end 145.085 95.555) (width 0.25) (layer "B.Cu") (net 61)))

